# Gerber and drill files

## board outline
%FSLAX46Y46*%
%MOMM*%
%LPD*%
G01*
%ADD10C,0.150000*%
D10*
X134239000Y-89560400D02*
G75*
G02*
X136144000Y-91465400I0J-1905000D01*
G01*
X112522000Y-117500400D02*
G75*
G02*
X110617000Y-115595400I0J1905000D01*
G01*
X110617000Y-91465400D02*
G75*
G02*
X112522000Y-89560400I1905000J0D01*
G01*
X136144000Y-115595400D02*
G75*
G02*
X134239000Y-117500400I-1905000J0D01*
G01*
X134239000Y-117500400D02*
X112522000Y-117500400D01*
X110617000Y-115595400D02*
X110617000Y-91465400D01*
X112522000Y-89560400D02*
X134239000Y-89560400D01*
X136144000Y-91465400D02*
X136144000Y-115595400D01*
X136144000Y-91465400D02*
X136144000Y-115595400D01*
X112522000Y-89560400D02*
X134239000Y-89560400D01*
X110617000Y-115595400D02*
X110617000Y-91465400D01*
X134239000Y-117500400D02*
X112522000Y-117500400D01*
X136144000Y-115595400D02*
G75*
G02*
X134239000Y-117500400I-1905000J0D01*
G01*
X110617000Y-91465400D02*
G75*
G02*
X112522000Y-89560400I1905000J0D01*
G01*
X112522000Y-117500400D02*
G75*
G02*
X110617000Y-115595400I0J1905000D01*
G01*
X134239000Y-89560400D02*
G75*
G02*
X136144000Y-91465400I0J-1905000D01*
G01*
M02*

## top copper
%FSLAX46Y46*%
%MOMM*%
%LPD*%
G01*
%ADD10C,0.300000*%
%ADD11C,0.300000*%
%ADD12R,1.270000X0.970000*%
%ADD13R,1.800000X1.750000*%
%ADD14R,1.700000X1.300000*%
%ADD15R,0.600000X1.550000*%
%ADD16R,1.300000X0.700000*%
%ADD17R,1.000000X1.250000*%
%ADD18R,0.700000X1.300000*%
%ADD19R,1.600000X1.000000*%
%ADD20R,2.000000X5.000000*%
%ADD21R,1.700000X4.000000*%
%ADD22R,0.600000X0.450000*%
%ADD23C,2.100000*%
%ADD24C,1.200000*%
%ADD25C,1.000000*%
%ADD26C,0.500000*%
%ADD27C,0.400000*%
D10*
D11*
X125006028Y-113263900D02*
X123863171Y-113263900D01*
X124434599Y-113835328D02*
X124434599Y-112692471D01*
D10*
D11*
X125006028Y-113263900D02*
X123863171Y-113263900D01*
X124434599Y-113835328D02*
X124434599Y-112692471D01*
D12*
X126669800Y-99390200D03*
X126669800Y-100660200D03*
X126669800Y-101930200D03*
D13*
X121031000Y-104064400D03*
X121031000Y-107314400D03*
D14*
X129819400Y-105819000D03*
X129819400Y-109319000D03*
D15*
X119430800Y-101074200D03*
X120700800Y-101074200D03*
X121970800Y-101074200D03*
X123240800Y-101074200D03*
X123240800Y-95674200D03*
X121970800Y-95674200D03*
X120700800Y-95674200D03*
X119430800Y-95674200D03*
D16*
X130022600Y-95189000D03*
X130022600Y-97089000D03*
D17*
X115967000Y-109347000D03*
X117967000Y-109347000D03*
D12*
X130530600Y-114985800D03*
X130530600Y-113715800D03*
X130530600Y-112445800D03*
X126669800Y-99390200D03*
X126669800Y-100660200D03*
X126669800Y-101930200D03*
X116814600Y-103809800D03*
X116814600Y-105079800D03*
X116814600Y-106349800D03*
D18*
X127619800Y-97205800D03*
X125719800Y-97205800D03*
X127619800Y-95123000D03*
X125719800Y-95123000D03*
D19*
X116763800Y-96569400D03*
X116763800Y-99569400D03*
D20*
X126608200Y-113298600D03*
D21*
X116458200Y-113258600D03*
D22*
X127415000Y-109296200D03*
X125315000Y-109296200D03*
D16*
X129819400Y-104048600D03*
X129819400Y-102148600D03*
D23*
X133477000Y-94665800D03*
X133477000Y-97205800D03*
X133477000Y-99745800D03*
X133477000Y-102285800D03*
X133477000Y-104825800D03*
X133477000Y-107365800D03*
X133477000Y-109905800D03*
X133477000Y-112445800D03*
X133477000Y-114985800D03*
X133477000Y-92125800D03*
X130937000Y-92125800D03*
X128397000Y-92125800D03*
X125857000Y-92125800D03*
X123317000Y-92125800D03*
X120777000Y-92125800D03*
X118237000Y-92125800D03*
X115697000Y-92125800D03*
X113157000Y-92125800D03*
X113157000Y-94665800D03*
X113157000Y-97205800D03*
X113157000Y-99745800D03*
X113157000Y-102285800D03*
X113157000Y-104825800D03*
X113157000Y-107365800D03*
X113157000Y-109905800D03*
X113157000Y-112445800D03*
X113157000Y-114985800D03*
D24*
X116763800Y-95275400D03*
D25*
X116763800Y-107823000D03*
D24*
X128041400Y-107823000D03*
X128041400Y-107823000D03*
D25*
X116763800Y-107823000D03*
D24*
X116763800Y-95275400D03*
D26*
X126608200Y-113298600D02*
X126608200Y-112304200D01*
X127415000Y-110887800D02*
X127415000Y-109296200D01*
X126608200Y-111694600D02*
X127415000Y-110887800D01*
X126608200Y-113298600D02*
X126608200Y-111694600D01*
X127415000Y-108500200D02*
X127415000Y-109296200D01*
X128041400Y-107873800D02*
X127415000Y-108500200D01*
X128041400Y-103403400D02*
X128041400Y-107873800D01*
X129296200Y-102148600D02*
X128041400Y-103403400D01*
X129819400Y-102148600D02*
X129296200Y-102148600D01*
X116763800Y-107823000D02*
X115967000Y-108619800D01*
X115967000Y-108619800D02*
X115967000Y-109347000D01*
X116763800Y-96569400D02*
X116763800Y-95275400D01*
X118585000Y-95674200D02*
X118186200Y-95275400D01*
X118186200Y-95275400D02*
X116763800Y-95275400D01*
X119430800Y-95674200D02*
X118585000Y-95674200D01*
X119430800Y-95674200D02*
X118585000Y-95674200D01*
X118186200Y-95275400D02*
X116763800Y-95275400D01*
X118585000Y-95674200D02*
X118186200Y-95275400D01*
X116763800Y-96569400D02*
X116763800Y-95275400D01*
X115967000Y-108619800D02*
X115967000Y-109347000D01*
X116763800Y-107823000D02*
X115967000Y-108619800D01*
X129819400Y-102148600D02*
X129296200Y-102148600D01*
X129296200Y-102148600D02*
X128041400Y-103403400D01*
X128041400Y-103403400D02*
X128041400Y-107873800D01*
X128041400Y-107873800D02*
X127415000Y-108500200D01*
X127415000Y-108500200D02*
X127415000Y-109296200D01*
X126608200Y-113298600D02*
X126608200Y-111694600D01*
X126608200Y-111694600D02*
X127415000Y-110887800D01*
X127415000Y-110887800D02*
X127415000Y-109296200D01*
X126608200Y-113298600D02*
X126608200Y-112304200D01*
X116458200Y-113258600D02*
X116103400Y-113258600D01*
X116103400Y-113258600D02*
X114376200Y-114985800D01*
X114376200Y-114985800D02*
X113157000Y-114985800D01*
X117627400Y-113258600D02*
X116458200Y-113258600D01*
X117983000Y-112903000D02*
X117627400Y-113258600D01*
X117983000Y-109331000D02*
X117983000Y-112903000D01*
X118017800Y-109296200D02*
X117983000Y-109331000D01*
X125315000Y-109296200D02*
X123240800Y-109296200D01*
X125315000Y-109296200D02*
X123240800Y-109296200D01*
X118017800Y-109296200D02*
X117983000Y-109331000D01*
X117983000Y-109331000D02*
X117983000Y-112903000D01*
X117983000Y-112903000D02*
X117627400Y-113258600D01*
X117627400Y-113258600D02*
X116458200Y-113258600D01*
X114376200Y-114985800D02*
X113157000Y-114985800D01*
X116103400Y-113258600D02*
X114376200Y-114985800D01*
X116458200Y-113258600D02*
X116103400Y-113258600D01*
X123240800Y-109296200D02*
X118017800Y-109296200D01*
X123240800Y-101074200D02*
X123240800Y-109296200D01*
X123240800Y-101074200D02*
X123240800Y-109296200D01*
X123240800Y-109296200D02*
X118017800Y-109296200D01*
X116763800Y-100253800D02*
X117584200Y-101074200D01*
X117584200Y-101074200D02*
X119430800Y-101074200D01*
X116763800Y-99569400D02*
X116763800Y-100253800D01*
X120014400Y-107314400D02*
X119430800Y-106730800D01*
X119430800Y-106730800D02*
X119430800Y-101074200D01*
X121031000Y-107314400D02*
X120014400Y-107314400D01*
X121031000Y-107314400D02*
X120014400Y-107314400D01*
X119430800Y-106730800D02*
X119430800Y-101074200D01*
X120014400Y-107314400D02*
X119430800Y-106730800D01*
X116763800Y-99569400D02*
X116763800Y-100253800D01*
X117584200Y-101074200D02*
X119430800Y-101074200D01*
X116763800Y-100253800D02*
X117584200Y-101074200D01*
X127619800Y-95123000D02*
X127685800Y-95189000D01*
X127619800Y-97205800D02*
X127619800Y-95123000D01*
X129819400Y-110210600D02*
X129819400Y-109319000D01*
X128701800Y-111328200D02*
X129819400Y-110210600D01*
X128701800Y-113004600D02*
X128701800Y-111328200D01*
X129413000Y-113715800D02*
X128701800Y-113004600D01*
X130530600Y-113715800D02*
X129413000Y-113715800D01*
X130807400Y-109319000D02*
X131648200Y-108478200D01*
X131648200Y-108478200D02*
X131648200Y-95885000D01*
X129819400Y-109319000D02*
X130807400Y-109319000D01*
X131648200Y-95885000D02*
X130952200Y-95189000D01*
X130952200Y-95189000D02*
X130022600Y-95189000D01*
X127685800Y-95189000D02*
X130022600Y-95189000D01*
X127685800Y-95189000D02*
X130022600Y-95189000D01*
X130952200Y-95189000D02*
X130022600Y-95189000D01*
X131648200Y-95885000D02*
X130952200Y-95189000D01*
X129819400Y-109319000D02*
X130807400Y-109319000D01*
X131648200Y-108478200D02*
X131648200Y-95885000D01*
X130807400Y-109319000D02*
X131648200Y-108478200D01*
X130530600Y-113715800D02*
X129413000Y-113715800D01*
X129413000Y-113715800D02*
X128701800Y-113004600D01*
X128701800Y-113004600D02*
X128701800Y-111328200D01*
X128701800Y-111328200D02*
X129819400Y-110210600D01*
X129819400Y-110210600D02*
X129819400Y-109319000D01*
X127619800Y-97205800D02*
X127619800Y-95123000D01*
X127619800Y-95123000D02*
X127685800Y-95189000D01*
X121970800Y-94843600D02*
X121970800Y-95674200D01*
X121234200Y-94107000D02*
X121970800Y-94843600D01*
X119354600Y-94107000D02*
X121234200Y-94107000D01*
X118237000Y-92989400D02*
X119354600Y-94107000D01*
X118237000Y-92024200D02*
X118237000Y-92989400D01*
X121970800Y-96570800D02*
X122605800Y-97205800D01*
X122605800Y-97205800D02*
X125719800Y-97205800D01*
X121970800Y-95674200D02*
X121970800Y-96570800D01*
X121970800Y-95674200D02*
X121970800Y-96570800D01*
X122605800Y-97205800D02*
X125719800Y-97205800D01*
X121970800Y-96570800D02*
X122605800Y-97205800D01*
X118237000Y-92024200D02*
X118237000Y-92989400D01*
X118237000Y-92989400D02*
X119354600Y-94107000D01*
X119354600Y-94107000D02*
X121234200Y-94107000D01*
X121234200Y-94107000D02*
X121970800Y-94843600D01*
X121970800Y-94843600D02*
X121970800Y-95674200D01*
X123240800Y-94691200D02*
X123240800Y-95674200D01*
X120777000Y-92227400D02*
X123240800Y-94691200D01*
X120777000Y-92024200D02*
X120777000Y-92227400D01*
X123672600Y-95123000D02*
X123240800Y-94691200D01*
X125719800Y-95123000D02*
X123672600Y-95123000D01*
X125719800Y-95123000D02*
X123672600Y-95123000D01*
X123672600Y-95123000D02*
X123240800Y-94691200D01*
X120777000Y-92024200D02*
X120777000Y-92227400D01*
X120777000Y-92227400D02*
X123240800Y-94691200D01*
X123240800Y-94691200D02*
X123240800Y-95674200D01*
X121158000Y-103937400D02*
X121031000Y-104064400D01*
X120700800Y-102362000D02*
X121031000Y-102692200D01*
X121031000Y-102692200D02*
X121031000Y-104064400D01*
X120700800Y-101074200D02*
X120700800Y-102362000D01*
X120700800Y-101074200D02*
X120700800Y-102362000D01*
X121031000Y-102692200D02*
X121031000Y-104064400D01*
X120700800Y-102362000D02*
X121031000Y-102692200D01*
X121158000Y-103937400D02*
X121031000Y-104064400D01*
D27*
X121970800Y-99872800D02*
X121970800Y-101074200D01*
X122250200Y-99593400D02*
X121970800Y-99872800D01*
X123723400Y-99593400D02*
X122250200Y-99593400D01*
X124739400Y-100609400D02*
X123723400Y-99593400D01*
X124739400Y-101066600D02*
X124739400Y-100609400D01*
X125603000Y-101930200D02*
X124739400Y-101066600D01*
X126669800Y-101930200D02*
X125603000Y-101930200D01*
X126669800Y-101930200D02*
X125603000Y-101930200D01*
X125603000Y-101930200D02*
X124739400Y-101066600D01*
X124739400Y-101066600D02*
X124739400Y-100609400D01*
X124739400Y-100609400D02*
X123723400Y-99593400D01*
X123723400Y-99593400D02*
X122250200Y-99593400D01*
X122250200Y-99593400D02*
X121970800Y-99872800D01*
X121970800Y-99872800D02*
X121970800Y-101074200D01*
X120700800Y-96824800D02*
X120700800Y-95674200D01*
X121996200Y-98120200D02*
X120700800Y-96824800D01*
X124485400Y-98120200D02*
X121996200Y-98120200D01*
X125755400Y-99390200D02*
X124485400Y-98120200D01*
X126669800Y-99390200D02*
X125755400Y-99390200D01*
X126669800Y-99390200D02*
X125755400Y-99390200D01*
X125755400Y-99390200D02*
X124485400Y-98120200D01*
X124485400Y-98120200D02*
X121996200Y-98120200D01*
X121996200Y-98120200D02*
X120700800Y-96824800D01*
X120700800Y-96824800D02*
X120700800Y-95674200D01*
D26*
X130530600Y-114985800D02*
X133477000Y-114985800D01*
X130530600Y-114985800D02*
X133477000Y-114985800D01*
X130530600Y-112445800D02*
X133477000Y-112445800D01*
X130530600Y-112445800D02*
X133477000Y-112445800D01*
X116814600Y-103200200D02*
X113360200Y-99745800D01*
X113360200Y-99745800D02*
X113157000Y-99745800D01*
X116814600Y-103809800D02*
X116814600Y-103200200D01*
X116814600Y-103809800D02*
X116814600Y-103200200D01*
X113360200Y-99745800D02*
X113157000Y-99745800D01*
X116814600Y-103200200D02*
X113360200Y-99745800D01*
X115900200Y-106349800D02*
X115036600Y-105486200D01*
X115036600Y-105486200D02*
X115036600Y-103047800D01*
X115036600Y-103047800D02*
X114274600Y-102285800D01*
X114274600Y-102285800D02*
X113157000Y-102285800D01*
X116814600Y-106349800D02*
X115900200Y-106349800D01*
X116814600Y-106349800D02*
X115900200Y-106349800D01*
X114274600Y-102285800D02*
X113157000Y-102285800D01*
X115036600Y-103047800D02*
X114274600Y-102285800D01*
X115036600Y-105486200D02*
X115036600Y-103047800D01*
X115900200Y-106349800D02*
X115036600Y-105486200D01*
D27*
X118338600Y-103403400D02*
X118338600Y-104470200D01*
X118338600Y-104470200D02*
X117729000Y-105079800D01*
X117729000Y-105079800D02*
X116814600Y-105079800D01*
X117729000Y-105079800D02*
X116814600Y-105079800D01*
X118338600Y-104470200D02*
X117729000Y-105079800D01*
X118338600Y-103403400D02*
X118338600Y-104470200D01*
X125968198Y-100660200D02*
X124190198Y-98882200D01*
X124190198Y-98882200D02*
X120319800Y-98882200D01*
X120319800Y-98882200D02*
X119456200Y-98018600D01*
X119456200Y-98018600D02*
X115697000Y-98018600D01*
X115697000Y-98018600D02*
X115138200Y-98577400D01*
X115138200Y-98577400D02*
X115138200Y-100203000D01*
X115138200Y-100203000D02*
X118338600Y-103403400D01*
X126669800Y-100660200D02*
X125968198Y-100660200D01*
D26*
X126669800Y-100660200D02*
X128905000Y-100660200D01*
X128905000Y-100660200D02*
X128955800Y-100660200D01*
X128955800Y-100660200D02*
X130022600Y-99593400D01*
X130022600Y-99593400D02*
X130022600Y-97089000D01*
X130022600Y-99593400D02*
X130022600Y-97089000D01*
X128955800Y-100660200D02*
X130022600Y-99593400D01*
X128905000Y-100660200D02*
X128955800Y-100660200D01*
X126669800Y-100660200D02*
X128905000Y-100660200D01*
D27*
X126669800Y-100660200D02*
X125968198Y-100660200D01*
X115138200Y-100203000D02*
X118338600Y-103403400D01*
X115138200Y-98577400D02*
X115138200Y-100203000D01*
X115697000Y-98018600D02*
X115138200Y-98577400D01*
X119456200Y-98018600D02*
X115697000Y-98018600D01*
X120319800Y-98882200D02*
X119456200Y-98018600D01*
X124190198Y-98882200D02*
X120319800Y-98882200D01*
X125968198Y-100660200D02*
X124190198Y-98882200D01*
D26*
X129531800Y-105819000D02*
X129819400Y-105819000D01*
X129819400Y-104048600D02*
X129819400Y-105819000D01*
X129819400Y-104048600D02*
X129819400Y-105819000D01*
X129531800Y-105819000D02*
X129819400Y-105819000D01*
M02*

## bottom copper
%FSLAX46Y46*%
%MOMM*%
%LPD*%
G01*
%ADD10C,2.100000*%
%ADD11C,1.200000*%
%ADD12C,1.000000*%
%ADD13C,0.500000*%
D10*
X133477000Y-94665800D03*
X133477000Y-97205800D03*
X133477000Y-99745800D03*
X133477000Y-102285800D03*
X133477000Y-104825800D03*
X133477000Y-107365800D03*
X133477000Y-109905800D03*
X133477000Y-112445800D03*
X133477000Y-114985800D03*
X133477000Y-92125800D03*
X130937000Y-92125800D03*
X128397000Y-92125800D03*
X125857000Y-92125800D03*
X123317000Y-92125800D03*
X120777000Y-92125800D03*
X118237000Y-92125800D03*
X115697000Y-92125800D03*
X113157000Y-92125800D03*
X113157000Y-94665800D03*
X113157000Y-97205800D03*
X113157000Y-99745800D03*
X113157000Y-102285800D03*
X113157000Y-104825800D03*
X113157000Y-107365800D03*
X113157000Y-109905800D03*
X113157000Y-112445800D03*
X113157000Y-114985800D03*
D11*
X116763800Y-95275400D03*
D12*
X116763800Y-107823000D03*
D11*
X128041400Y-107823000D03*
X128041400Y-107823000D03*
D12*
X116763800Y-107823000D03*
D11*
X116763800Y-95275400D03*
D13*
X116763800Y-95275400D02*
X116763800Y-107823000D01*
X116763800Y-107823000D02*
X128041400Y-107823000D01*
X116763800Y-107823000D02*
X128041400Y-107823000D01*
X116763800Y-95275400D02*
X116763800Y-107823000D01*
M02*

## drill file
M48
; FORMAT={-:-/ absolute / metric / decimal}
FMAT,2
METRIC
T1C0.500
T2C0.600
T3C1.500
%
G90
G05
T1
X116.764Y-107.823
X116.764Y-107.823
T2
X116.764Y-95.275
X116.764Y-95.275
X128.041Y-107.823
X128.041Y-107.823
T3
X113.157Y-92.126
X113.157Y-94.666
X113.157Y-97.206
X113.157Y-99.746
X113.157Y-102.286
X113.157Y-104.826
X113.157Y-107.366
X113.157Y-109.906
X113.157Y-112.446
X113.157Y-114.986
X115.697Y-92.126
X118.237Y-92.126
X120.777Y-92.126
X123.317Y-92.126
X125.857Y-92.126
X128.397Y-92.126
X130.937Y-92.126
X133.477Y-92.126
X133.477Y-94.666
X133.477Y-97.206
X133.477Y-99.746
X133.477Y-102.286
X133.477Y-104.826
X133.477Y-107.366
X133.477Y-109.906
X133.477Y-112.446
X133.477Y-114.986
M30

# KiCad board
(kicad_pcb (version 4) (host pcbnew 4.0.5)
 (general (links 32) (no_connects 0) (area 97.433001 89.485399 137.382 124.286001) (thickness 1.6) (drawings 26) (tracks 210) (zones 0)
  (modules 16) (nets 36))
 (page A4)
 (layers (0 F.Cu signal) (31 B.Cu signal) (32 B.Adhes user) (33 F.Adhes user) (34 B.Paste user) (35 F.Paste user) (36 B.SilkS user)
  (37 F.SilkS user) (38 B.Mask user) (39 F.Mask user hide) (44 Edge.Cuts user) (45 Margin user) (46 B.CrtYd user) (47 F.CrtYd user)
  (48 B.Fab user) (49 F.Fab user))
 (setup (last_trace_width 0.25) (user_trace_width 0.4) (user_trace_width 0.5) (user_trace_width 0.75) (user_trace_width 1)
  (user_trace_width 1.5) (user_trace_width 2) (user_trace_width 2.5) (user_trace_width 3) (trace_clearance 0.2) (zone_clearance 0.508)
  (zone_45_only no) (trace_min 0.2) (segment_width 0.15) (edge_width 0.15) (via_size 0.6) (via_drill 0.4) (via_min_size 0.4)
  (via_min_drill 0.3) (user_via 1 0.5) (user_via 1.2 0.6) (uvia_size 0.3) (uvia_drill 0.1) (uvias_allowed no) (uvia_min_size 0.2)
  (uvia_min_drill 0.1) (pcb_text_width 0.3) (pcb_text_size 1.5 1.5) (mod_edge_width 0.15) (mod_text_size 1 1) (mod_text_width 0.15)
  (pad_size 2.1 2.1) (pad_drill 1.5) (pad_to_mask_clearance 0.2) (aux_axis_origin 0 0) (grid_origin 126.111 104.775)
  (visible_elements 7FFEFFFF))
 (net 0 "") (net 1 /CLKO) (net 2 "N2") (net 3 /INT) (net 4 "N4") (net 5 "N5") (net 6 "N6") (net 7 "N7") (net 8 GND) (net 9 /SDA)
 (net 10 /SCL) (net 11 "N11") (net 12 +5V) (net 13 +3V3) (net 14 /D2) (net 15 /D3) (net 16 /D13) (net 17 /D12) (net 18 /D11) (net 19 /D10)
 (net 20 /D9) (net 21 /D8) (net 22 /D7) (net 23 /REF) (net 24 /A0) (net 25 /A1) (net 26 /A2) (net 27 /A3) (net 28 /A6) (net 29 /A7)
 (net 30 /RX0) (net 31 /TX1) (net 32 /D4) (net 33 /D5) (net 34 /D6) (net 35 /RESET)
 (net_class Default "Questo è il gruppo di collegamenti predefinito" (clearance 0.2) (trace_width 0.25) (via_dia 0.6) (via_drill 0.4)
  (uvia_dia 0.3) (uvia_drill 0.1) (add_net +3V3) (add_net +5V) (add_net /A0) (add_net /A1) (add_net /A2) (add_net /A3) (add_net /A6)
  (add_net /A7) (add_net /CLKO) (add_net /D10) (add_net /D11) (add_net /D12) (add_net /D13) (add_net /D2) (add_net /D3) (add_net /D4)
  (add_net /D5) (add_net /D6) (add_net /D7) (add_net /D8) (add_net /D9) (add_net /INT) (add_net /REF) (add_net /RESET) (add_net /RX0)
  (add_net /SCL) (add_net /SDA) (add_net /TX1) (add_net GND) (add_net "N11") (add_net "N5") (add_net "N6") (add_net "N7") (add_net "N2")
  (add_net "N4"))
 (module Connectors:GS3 (layer F.Cu) (at 126.6698 100.6602)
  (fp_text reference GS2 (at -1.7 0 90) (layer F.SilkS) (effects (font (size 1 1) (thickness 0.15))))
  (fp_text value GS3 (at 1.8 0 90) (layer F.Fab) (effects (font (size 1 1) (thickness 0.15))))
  (pad 1 smd rect (at 0 -1.27) (size 1.27 0.97) (layers F.Cu F.Paste F.Mask) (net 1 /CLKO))
  (pad 2 smd rect (at 0 0) (size 1.27 0.97) (layers F.Cu F.Paste F.Mask) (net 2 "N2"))
  (pad 3 smd rect (at 0 1.27) (size 1.27 0.97) (layers F.Cu F.Paste F.Mask) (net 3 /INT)))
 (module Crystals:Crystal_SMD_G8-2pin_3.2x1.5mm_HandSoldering (layer F.Cu) (at 121.031 105.6894 270)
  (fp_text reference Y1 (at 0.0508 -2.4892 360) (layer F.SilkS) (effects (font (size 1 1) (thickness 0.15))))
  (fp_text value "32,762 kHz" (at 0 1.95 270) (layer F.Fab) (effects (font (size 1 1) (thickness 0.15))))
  (pad 1 smd rect (at -1.625 0 270) (size 1.75 1.8) (layers F.Cu F.Paste F.Mask) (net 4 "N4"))
  (pad 2 smd rect (at 1.625 0 270) (size 1.75 1.8) (layers F.Cu F.Paste F.Mask) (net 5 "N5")))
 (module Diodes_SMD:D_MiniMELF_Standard (layer F.Cu) (at 129.8194 107.569 270)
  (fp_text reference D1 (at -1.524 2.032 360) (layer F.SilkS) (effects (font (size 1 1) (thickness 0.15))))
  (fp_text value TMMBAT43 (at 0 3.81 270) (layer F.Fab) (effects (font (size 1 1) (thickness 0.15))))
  (pad 1 smd rect (at -1.75 0 270) (size 1.3 1.7) (layers F.Cu F.Paste F.Mask) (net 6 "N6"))
  (pad 2 smd rect (at 1.75 0 270) (size 1.3 1.7) (layers F.Cu F.Paste F.Mask) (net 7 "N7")))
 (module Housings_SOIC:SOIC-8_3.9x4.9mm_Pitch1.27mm (layer F.Cu) (at 121.3358 98.3742 90)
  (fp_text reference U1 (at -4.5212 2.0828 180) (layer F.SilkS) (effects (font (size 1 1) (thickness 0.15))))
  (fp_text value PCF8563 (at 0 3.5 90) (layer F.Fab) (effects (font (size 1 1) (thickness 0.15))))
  (pad 1 smd rect (at -2.7 -1.905 90) (size 1.55 0.6) (layers F.Cu F.Paste F.Mask) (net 5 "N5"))
  (pad 2 smd rect (at -2.7 -0.635 90) (size 1.55 0.6) (layers F.Cu F.Paste F.Mask) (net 4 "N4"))
  (pad 3 smd rect (at -2.7 0.635 90) (size 1.55 0.6) (layers F.Cu F.Paste F.Mask) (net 3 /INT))
  (pad 4 smd rect (at -2.7 1.905 90) (size 1.55 0.6) (layers F.Cu F.Paste F.Mask) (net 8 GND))
  (pad 5 smd rect (at 2.7 1.905 90) (size 1.55 0.6) (layers F.Cu F.Paste F.Mask) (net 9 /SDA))
  (pad 6 smd rect (at 2.7 0.635 90) (size 1.55 0.6) (layers F.Cu F.Paste F.Mask) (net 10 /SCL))
  (pad 7 smd rect (at 2.7 -0.635 90) (size 1.55 0.6) (layers F.Cu F.Paste F.Mask) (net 1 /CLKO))
  (pad 8 smd rect (at 2.7 -1.905 90) (size 1.55 0.6) (layers F.Cu F.Paste F.Mask) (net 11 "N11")))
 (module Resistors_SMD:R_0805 (layer F.Cu) (at 130.0226 96.139 270)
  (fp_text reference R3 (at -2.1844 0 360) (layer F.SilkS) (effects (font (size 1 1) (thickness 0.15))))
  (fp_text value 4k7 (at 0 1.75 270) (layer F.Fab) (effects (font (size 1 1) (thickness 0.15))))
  (pad 1 smd rect (at -0.95 0 270) (size 0.7 1.3) (layers F.Cu F.Paste F.Mask) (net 7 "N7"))
  (pad 2 smd rect (at 0.95 0 270) (size 0.7 1.3) (layers F.Cu F.Paste F.Mask) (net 2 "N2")))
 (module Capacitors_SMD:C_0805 (layer F.Cu) (at 116.967 109.347)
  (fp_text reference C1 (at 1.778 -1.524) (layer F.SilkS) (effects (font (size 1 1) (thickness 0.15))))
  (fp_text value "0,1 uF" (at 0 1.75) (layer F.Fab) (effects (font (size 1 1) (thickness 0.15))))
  (pad 1 smd rect (at -1 0) (size 1 1.25) (layers F.Cu F.Paste F.Mask) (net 11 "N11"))
  (pad 2 smd rect (at 1 0) (size 1 1.25) (layers F.Cu F.Paste F.Mask) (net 8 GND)))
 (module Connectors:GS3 (layer F.Cu) (at 130.5306 113.7158 180)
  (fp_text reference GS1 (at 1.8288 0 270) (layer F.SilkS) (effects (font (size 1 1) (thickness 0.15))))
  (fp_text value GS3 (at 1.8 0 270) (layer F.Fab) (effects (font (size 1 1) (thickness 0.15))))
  (pad 1 smd rect (at 0 -1.27 180) (size 1.27 0.97) (layers F.Cu F.Paste F.Mask) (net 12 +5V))
  (pad 2 smd rect (at 0 0 180) (size 1.27 0.97) (layers F.Cu F.Paste F.Mask) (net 7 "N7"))
  (pad 3 smd rect (at 0 1.27 180) (size 1.27 0.97) (layers F.Cu F.Paste F.Mask) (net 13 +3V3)))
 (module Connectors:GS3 (layer F.Cu) (at 126.6698 100.6602)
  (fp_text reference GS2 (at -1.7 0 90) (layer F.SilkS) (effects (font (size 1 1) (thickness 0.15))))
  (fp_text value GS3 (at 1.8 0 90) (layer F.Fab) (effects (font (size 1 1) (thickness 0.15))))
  (pad 1 smd rect (at 0 -1.27) (size 1.27 0.97) (layers F.Cu F.Paste F.Mask) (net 1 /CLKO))
  (pad 2 smd rect (at 0 0) (size 1.27 0.97) (layers F.Cu F.Paste F.Mask) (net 2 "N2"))
  (pad 3 smd rect (at 0 1.27) (size 1.27 0.97) (layers F.Cu F.Paste F.Mask) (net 3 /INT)))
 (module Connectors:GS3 (layer F.Cu) (at 116.8146 105.0798)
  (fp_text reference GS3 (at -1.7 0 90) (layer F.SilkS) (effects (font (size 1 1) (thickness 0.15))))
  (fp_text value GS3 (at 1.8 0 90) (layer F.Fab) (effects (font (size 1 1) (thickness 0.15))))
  (pad 1 smd rect (at 0 -1.27) (size 1.27 0.97) (layers F.Cu F.Paste F.Mask) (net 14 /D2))
  (pad 2 smd rect (at 0 0) (size 1.27 0.97) (layers F.Cu F.Paste F.Mask) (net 2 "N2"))
  (pad 3 smd rect (at 0 1.27) (size 1.27 0.97) (layers F.Cu F.Paste F.Mask) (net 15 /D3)))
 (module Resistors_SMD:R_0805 (layer F.Cu) (at 126.6698 97.2058 180)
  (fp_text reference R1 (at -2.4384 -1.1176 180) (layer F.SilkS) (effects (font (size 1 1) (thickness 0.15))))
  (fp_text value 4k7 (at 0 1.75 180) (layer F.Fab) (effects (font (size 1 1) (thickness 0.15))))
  (pad 1 smd rect (at -0.95 0 180) (size 0.7 1.3) (layers F.Cu F.Paste F.Mask) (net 7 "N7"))
  (pad 2 smd rect (at 0.95 0 180) (size 0.7 1.3) (layers F.Cu F.Paste F.Mask) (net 10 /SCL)))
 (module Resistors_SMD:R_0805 (layer F.Cu) (at 126.6698 95.123 180)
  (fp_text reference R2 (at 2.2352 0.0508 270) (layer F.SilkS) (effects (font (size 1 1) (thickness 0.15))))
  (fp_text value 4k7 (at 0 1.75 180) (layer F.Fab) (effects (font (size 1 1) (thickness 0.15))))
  (pad 1 smd rect (at -0.95 0 180) (size 0.7 1.3) (layers F.Cu F.Paste F.Mask) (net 7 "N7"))
  (pad 2 smd rect (at 0.95 0 180) (size 0.7 1.3) (layers F.Cu F.Paste F.Mask) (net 9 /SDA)))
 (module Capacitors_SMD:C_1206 (layer F.Cu) (at 116.7638 98.0694 270)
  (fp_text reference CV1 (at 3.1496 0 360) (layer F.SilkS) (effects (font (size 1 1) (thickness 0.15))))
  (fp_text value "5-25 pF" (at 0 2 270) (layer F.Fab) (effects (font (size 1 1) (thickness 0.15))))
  (pad 1 smd rect (at -1.5 0 270) (size 1 1.6) (layers F.Cu F.Paste F.Mask) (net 11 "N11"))
  (pad 2 smd rect (at 1.5 0 270) (size 1 1.6) (layers F.Cu F.Paste F.Mask) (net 5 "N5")))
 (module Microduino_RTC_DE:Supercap (layer F.Cu) (at 121.4882 113.2586 180)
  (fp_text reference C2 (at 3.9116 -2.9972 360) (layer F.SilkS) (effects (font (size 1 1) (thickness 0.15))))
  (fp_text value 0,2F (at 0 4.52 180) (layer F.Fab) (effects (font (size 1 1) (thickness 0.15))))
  (pad 1 smd rect (at -5.12 -0.04 180) (size 2 5) (layers F.Cu F.Paste F.Mask) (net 11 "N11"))
  (pad 2 smd rect (at 5.03 0 180) (size 1.7 4) (layers F.Cu F.Mask) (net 8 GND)))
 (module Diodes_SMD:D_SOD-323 (layer F.Cu) (at 126.365 109.2962 180)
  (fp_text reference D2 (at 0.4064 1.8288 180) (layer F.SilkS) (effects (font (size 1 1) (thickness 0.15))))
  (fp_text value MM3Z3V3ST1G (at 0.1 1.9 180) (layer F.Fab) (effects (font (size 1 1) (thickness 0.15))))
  (pad 1 smd rect (at -1.05 0 180) (size 0.6 0.45) (layers F.Cu F.Paste F.Mask) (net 11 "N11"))
  (pad 2 smd rect (at 1.05 0 180) (size 0.6 0.45) (layers F.Cu F.Paste F.Mask) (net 8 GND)))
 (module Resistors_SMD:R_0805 (layer F.Cu) (at 129.8194 103.0986 90)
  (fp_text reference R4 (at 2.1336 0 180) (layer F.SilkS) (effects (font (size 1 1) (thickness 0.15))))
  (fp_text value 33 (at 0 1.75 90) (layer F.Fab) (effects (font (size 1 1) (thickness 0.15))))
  (pad 1 smd rect (at -0.95 0 90) (size 0.7 1.3) (layers F.Cu F.Paste F.Mask) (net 6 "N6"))
  (pad 2 smd rect (at 0.95 0 90) (size 0.7 1.3) (layers F.Cu F.Paste F.Mask) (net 11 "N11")))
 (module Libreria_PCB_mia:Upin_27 (layer B.Cu) (at 133.477 114.9858 180)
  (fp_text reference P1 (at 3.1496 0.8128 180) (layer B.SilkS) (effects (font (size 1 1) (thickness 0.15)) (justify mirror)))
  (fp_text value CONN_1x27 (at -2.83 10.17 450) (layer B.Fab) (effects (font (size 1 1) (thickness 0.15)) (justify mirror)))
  (pad 9 thru_hole circle (at 0 20.32 180) (size 2.1 2.1) (drill 1.5) (layers *.Cu *.Mask) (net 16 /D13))
  (pad 8 thru_hole circle (at 0 17.78 180) (size 2.1 2.1) (drill 1.5) (layers *.Cu *.Mask) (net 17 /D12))
  (pad 7 thru_hole circle (at 0 15.24 180) (size 2.1 2.1) (drill 1.5) (layers *.Cu *.Mask) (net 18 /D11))
  (pad 6 thru_hole circle (at 0 12.7 180) (size 2.1 2.1) (drill 1.5) (layers *.Cu *.Mask) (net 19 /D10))
  (pad 5 thru_hole circle (at 0 10.16 180) (size 2.1 2.1) (drill 1.5) (layers *.Cu *.Mask) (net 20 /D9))
  (pad 4 thru_hole circle (at 0 7.62 180) (size 2.1 2.1) (drill 1.5) (layers *.Cu *.Mask) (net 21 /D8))
  (pad 3 thru_hole circle (at 0 5.08 180) (size 2.1 2.1) (drill 1.5) (layers *.Cu *.Mask) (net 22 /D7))
  (pad 2 thru_hole circle (at 0 2.54 180) (size 2.1 2.1) (drill 1.5) (layers *.Cu *.Mask) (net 13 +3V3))
  (pad 1 thru_hole circle (at 0 0 180) (size 2.1 2.1) (drill 1.5) (layers *.Cu *.Mask) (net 12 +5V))
  (pad 10 thru_hole circle (at 0 22.86 180) (size 2.1 2.1) (drill 1.5) (layers *.Cu *.Mask) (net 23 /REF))
  (pad 11 thru_hole circle (at 2.54 22.86 180) (size 2.1 2.1) (drill 1.5) (layers *.Cu *.Mask) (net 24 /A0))
  (pad 12 thru_hole circle (at 5.08 22.86 180) (size 2.1 2.1) (drill 1.5) (layers *.Cu *.Mask) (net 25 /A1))
  (pad 13 thru_hole circle (at 7.62 22.86 180) (size 2.1 2.1) (drill 1.5) (layers *.Cu *.Mask) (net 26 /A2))
  (pad 14 thru_hole circle (at 10.16 22.86 180) (size 2.1 2.1) (drill 1.5) (layers *.Cu *.Mask) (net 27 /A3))
  (pad 15 thru_hole circle (at 12.7 22.86 180) (size 2.1 2.1) (drill 1.5) (layers *.Cu *.Mask) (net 9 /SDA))
  (pad 16 thru_hole circle (at 15.24 22.86 180) (size 2.1 2.1) (drill 1.5) (layers *.Cu *.Mask) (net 10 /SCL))
  (pad 17 thru_hole circle (at 17.78 22.86 180) (size 2.1 2.1) (drill 1.5) (layers *.Cu *.Mask) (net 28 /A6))
  (pad 18 thru_hole circle (at 20.32 22.86 180) (size 2.1 2.1) (drill 1.5) (layers *.Cu *.Mask) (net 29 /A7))
  (pad 19 thru_hole circle (at 20.32 20.32 180) (size 2.1 2.1) (drill 1.5) (layers *.Cu *.Mask) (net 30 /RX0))
  (pad 20 thru_hole circle (at 20.32 17.78 180) (size 2.1 2.1) (drill 1.5) (layers *.Cu *.Mask) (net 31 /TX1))
  (pad 21 thru_hole circle (at 20.32 15.24 180) (size 2.1 2.1) (drill 1.5) (layers *.Cu *.Mask) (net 14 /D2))
  (pad 22 thru_hole circle (at 20.32 12.7 180) (size 2.1 2.1) (drill 1.5) (layers *.Cu *.Mask) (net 15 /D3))
  (pad 23 thru_hole circle (at 20.32 10.16 180) (size 2.1 2.1) (drill 1.5) (layers *.Cu *.Mask) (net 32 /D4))
  (pad 24 thru_hole circle (at 20.32 7.62 180) (size 2.1 2.1) (drill 1.5) (layers *.Cu *.Mask) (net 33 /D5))
  (pad 25 thru_hole circle (at 20.32 5.08 180) (size 2.1 2.1) (drill 1.5) (layers *.Cu *.Mask) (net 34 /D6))
  (pad 26 thru_hole circle (at 20.32 2.54 180) (size 2.1 2.1) (drill 1.5) (layers *.Cu *.Mask) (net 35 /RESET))
  (pad 27 thru_hole circle (at 20.32 0 180) (size 2.1 2.1) (drill 1.5) (layers *.Cu *.Mask) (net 8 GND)))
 (gr_arc (start 134.239 91.4654) (end 134.239 89.5604) (angle 90) (layer Edge.Cuts) (width 0.15))
 (gr_arc (start 112.522 115.5954) (end 112.522 117.5004) (angle 90) (layer Edge.Cuts) (width 0.15))
 (gr_arc (start 112.522 91.4654) (end 110.617 91.4654) (angle 90) (layer Edge.Cuts) (width 0.15))
 (gr_arc (start 134.239 115.5954) (end 136.144 115.5954) (angle 90) (layer Edge.Cuts) (width 0.15))
 (gr_line (start 134.239 117.5004) (end 112.522 117.5004) (angle 90) (layer Edge.Cuts) (width 0.15))
 (gr_line (start 110.617 115.5954) (end 110.617 91.4654) (angle 90) (layer Edge.Cuts) (width 0.15))
 (gr_line (start 112.522 89.5604) (end 134.239 89.5604) (angle 90) (layer Edge.Cuts) (width 0.15))
 (gr_line (start 136.144 91.4654) (end 136.144 115.5954) (angle 90) (layer Edge.Cuts) (width 0.15))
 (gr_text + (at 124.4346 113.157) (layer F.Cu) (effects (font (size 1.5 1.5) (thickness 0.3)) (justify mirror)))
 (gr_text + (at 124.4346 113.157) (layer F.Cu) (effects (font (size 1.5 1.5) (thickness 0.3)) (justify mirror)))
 (gr_line (start 136.144 91.4654) (end 136.144 115.5954) (angle 90) (layer Edge.Cuts) (width 0.15))
 (gr_line (start 112.522 89.5604) (end 134.239 89.5604) (angle 90) (layer Edge.Cuts) (width 0.15))
 (gr_line (start 110.617 115.5954) (end 110.617 91.4654) (angle 90) (layer Edge.Cuts) (width 0.15))
 (gr_line (start 134.239 117.5004) (end 112.522 117.5004) (angle 90) (layer Edge.Cuts) (width 0.15))
 (gr_arc (start 134.239 115.5954) (end 136.144 115.5954) (angle 90) (layer Edge.Cuts) (width 0.15))
 (gr_arc (start 112.522 91.4654) (end 110.617 91.4654) (angle 90) (layer Edge.Cuts) (width 0.15))
 (gr_arc (start 112.522 115.5954) (end 112.522 117.5004) (angle 90) (layer Edge.Cuts) (width 0.15))
 (gr_arc (start 134.239 91.4654) (end 134.239 89.5604) (angle 90) (layer Edge.Cuts) (width 0.15))
 (segment (start 126.6082 113.2986) (end 126.6082 112.3042) (width 0.5) (layer F.Cu) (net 11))
 (segment (start 127.415 110.8878) (end 127.415 109.2962) (width 0.5) (layer F.Cu) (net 11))
 (segment (start 126.6082 111.6946) (end 127.415 110.8878) (width 0.5) (layer F.Cu) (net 11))
 (segment (start 126.6082 113.2986) (end 126.6082 111.6946) (width 0.5) (layer F.Cu) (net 11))
 (segment (start 127.415 108.5002) (end 127.415 109.2962) (width 0.5) (layer F.Cu) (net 11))
 (segment (start 128.0414 107.8738) (end 127.415 108.5002) (width 0.5) (layer F.Cu) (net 11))
 (segment (start 128.0414 103.4034) (end 128.0414 107.8738) (width 0.5) (layer F.Cu) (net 11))
 (segment (start 129.2962 102.1486) (end 128.0414 103.4034) (width 0.5) (layer F.Cu) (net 11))
 (segment (start 129.8194 102.1486) (end 129.2962 102.1486) (width 0.5) (layer F.Cu) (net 11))
 (via (at 116.7638 95.2754) (size 1.2) (drill 0.6) (layers F.Cu B.Cu) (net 11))
 (segment (start 116.7638 95.2754) (end 116.7638 107.823) (width 0.5) (layer B.Cu) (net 11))
 (via (at 116.7638 107.823) (size 1) (drill 0.5) (layers F.Cu B.Cu) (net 11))
 (segment (start 116.7638 107.823) (end 115.967 108.6198) (width 0.5) (layer F.Cu) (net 11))
 (segment (start 115.967 108.6198) (end 115.967 109.347) (width 0.5) (layer F.Cu) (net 11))
 (segment (start 116.7638 96.5694) (end 116.7638 95.2754) (width 0.5) (layer F.Cu) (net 11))
 (segment (start 118.585 95.6742) (end 118.1862 95.2754) (width 0.5) (layer F.Cu) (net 11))
 (segment (start 118.1862 95.2754) (end 116.7638 95.2754) (width 0.5) (layer F.Cu) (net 11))
 (segment (start 119.4308 95.6742) (end 118.585 95.6742) (width 0.5) (layer F.Cu) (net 11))
 (via (at 128.0414 107.823) (size 1.2) (drill 0.6) (layers F.Cu B.Cu) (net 11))
 (segment (start 116.7638 107.823) (end 128.0414 107.823) (width 0.5) (layer B.Cu) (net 11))
 (segment (start 116.7638 107.823) (end 128.0414 107.823) (width 0.5) (layer B.Cu) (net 11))
 (via (at 128.0414 107.823) (size 1.2) (drill 0.6) (layers F.Cu B.Cu) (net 11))
 (segment (start 119.4308 95.6742) (end 118.585 95.6742) (width 0.5) (layer F.Cu) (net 11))
 (segment (start 118.1862 95.2754) (end 116.7638 95.2754) (width 0.5) (layer F.Cu) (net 11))
 (segment (start 118.585 95.6742) (end 118.1862 95.2754) (width 0.5) (layer F.Cu) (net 11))
 (segment (start 116.7638 96.5694) (end 116.7638 95.2754) (width 0.5) (layer F.Cu) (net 11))
 (segment (start 115.967 108.6198) (end 115.967 109.347) (width 0.5) (layer F.Cu) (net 11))
 (segment (start 116.7638 107.823) (end 115.967 108.6198) (width 0.5) (layer F.Cu) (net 11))
 (via (at 116.7638 107.823) (size 1) (drill 0.5) (layers F.Cu B.Cu) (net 11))
 (segment (start 116.7638 95.2754) (end 116.7638 107.823) (width 0.5) (layer B.Cu) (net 11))
 (via (at 116.7638 95.2754) (size 1.2) (drill 0.6) (layers F.Cu B.Cu) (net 11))
 (segment (start 129.8194 102.1486) (end 129.2962 102.1486) (width 0.5) (layer F.Cu) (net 11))
 (segment (start 129.2962 102.1486) (end 128.0414 103.4034) (width 0.5) (layer F.Cu) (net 11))
 (segment (start 128.0414 103.4034) (end 128.0414 107.8738) (width 0.5) (layer F.Cu) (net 11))
 (segment (start 128.0414 107.8738) (end 127.415 108.5002) (width 0.5) (layer F.Cu) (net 11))
 (segment (start 127.415 108.5002) (end 127.415 109.2962) (width 0.5) (layer F.Cu) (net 11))
 (segment (start 126.6082 113.2986) (end 126.6082 111.6946) (width 0.5) (layer F.Cu) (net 11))
 (segment (start 126.6082 111.6946) (end 127.415 110.8878) (width 0.5) (layer F.Cu) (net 11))
 (segment (start 127.415 110.8878) (end 127.415 109.2962) (width 0.5) (layer F.Cu) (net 11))
 (segment (start 126.6082 113.2986) (end 126.6082 112.3042) (width 0.5) (layer F.Cu) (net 11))
 (segment (start 116.4582 113.2586) (end 116.1034 113.2586) (width 0.5) (layer F.Cu) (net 8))
 (segment (start 116.1034 113.2586) (end 114.3762 114.9858) (width 0.5) (layer F.Cu) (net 8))
 (segment (start 114.3762 114.9858) (end 113.157 114.9858) (width 0.5) (layer F.Cu) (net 8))
 (segment (start 117.6274 113.2586) (end 116.4582 113.2586) (width 0.5) (layer F.Cu) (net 8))
 (segment (start 117.983 112.903) (end 117.6274 113.2586) (width 0.5) (layer F.Cu) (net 8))
 (segment (start 117.983 109.331) (end 117.983 112.903) (width 0.5) (layer F.Cu) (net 8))
 (segment (start 118.0178 109.2962) (end 117.983 109.331) (width 0.5) (layer F.Cu) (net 8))
 (segment (start 125.315 109.2962) (end 123.2408 109.2962) (width 0.5) (layer F.Cu) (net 8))
 (segment (start 125.315 109.2962) (end 123.2408 109.2962) (width 0.5) (layer F.Cu) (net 8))
 (segment (start 118.0178 109.2962) (end 117.983 109.331) (width 0.5) (layer F.Cu) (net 8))
 (segment (start 117.983 109.331) (end 117.983 112.903) (width 0.5) (layer F.Cu) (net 8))
 (segment (start 117.983 112.903) (end 117.6274 113.2586) (width 0.5) (layer F.Cu) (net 8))
 (segment (start 117.6274 113.2586) (end 116.4582 113.2586) (width 0.5) (layer F.Cu) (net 8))
 (segment (start 114.3762 114.9858) (end 113.157 114.9858) (width 0.5) (layer F.Cu) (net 8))
 (segment (start 116.1034 113.2586) (end 114.3762 114.9858) (width 0.5) (layer F.Cu) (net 8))
 (segment (start 116.4582 113.2586) (end 116.1034 113.2586) (width 0.5) (layer F.Cu) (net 8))
 (segment (start 123.2408 109.2962) (end 118.0178 109.2962) (width 0.5) (layer F.Cu) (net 8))
 (segment (start 123.2408 101.0742) (end 123.2408 109.2962) (width 0.5) (layer F.Cu) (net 8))
 (segment (start 123.2408 101.0742) (end 123.2408 109.2962) (width 0.5) (layer F.Cu) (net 8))
 (segment (start 123.2408 109.2962) (end 118.0178 109.2962) (width 0.5) (layer F.Cu) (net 8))
 (segment (start 116.7638 100.2538) (end 117.5842 101.0742) (width 0.5) (layer F.Cu) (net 5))
 (segment (start 117.5842 101.0742) (end 119.4308 101.0742) (width 0.5) (layer F.Cu) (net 5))
 (segment (start 116.7638 99.5694) (end 116.7638 100.2538) (width 0.5) (layer F.Cu) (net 5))
 (segment (start 120.0144 107.3144) (end 119.4308 106.7308) (width 0.5) (layer F.Cu) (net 5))
 (segment (start 119.4308 106.7308) (end 119.4308 101.0742) (width 0.5) (layer F.Cu) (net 5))
 (segment (start 121.031 107.3144) (end 120.0144 107.3144) (width 0.5) (layer F.Cu) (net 5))
 (segment (start 121.031 107.3144) (end 120.0144 107.3144) (width 0.5) (layer F.Cu) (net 5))
 (segment (start 119.4308 106.7308) (end 119.4308 101.0742) (width 0.5) (layer F.Cu) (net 5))
 (segment (start 120.0144 107.3144) (end 119.4308 106.7308) (width 0.5) (layer F.Cu) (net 5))
 (segment (start 116.7638 99.5694) (end 116.7638 100.2538) (width 0.5) (layer F.Cu) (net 5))
 (segment (start 117.5842 101.0742) (end 119.4308 101.0742) (width 0.5) (layer F.Cu) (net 5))
 (segment (start 116.7638 100.2538) (end 117.5842 101.0742) (width 0.5) (layer F.Cu) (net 5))
 (segment (start 127.6198 95.123) (end 127.6858 95.189) (width 0.5) (layer F.Cu) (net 7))
 (segment (start 127.6198 97.2058) (end 127.6198 95.123) (width 0.5) (layer F.Cu) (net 7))
 (segment (start 129.8194 110.2106) (end 129.8194 109.319) (width 0.5) (layer F.Cu) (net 7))
 (segment (start 128.7018 111.3282) (end 129.8194 110.2106) (width 0.5) (layer F.Cu) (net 7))
 (segment (start 128.7018 113.0046) (end 128.7018 111.3282) (width 0.5) (layer F.Cu) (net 7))
 (segment (start 129.413 113.7158) (end 128.7018 113.0046) (width 0.5) (layer F.Cu) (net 7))
 (segment (start 130.5306 113.7158) (end 129.413 113.7158) (width 0.5) (layer F.Cu) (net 7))
 (segment (start 130.8074 109.319) (end 131.6482 108.4782) (width 0.5) (layer F.Cu) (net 7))
 (segment (start 131.6482 108.4782) (end 131.6482 95.885) (width 0.5) (layer F.Cu) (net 7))
 (segment (start 129.8194 109.319) (end 130.8074 109.319) (width 0.5) (layer F.Cu) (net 7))
 (segment (start 131.6482 95.885) (end 130.9522 95.189) (width 0.5) (layer F.Cu) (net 7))
 (segment (start 130.9522 95.189) (end 130.0226 95.189) (width 0.5) (layer F.Cu) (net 7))
 (segment (start 127.6858 95.189) (end 130.0226 95.189) (width 0.5) (layer F.Cu) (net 7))
 (segment (start 127.6858 95.189) (end 130.0226 95.189) (width 0.5) (layer F.Cu) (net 7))
 (segment (start 130.9522 95.189) (end 130.0226 95.189) (width 0.5) (layer F.Cu) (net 7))
 (segment (start 131.6482 95.885) (end 130.9522 95.189) (width 0.5) (layer F.Cu) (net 7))
 (segment (start 129.8194 109.319) (end 130.8074 109.319) (width 0.5) (layer F.Cu) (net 7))
 (segment (start 131.6482 108.4782) (end 131.6482 95.885) (width 0.5) (layer F.Cu) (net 7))
 (segment (start 130.8074 109.319) (end 131.6482 108.4782) (width 0.5) (layer F.Cu) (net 7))
 (segment (start 130.5306 113.7158) (end 129.413 113.7158) (width 0.5) (layer F.Cu) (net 7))
 (segment (start 129.413 113.7158) (end 128.7018 113.0046) (width 0.5) (layer F.Cu) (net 7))
 (segment (start 128.7018 113.0046) (end 128.7018 111.3282) (width 0.5) (layer F.Cu) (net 7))
 (segment (start 128.7018 111.3282) (end 129.8194 110.2106) (width 0.5) (layer F.Cu) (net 7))
 (segment (start 129.8194 110.2106) (end 129.8194 109.319) (width 0.5) (layer F.Cu) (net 7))
 (segment (start 127.6198 97.2058) (end 127.6198 95.123) (width 0.5) (layer F.Cu) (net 7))
 (segment (start 127.6198 95.123) (end 127.6858 95.189) (width 0.5) (layer F.Cu) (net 7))
 (segment (start 121.9708 94.8436) (end 121.9708 95.6742) (width 0.5) (layer F.Cu) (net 10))
 (segment (start 121.2342 94.107) (end 121.9708 94.8436) (width 0.5) (layer F.Cu) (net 10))
 (segment (start 119.3546 94.107) (end 121.2342 94.107) (width 0.5) (layer F.Cu) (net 10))
 (segment (start 118.237 92.9894) (end 119.3546 94.107) (width 0.5) (layer F.Cu) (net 10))
 (segment (start 118.237 92.0242) (end 118.237 92.9894) (width 0.5) (layer F.Cu) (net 10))
 (segment (start 121.9708 96.5708) (end 122.6058 97.2058) (width 0.5) (layer F.Cu) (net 10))
 (segment (start 122.6058 97.2058) (end 125.7198 97.2058) (width 0.5) (layer F.Cu) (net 10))
 (segment (start 121.9708 95.6742) (end 121.9708 96.5708) (width 0.5) (layer F.Cu) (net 10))
 (segment (start 121.9708 95.6742) (end 121.9708 96.5708) (width 0.5) (layer F.Cu) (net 10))
 (segment (start 122.6058 97.2058) (end 125.7198 97.2058) (width 0.5) (layer F.Cu) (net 10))
 (segment (start 121.9708 96.5708) (end 122.6058 97.2058) (width 0.5) (layer F.Cu) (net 10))
 (segment (start 118.237 92.0242) (end 118.237 92.9894) (width 0.5) (layer F.Cu) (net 10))
 (segment (start 118.237 92.9894) (end 119.3546 94.107) (width 0.5) (layer F.Cu) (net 10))
 (segment (start 119.3546 94.107) (end 121.2342 94.107) (width 0.5) (layer F.Cu) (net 10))
 (segment (start 121.2342 94.107) (end 121.9708 94.8436) (width 0.5) (layer F.Cu) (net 10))
 (segment (start 121.9708 94.8436) (end 121.9708 95.6742) (width 0.5) (layer F.Cu) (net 10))
 (segment (start 123.2408 94.6912) (end 123.2408 95.6742) (width 0.5) (layer F.Cu) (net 9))
 (segment (start 120.777 92.2274) (end 123.2408 94.6912) (width 0.5) (layer F.Cu) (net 9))
 (segment (start 120.777 92.0242) (end 120.777 92.2274) (width 0.5) (layer F.Cu) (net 9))
 (segment (start 123.6726 95.123) (end 123.2408 94.6912) (width 0.5) (layer F.Cu) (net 9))
 (segment (start 125.7198 95.123) (end 123.6726 95.123) (width 0.5) (layer F.Cu) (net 9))
 (segment (start 125.7198 95.123) (end 123.6726 95.123) (width 0.5) (layer F.Cu) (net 9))
 (segment (start 123.6726 95.123) (end 123.2408 94.6912) (width 0.5) (layer F.Cu) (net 9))
 (segment (start 120.777 92.0242) (end 120.777 92.2274) (width 0.5) (layer F.Cu) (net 9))
 (segment (start 120.777 92.2274) (end 123.2408 94.6912) (width 0.5) (layer F.Cu) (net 9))
 (segment (start 123.2408 94.6912) (end 123.2408 95.6742) (width 0.5) (layer F.Cu) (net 9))
 (segment (start 121.158 103.9374) (end 121.031 104.0644) (width 0.5) (layer F.Cu) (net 4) (status 30))
 (segment (start 120.7008 102.362) (end 121.031 102.6922) (width 0.5) (layer F.Cu) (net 4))
 (segment (start 121.031 102.6922) (end 121.031 104.0644) (width 0.5) (layer F.Cu) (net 4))
 (segment (start 120.7008 101.0742) (end 120.7008 102.362) (width 0.5) (layer F.Cu) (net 4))
 (segment (start 120.7008 101.0742) (end 120.7008 102.362) (width 0.5) (layer F.Cu) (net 4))
 (segment (start 121.031 102.6922) (end 121.031 104.0644) (width 0.5) (layer F.Cu) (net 4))
 (segment (start 120.7008 102.362) (end 121.031 102.6922) (width 0.5) (layer F.Cu) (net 4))
 (segment (start 121.158 103.9374) (end 121.031 104.0644) (width 0.5) (layer F.Cu) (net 4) (status 30))
 (segment (start 121.9708 99.8728) (end 121.9708 101.0742) (width 0.4) (layer F.Cu) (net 3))
 (segment (start 122.2502 99.5934) (end 121.9708 99.8728) (width 0.4) (layer F.Cu) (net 3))
 (segment (start 123.7234 99.5934) (end 122.2502 99.5934) (width 0.4) (layer F.Cu) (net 3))
 (segment (start 124.7394 100.6094) (end 123.7234 99.5934) (width 0.4) (layer F.Cu) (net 3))
 (segment (start 124.7394 101.0666) (end 124.7394 100.6094) (width 0.4) (layer F.Cu) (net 3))
 (segment (start 125.603 101.9302) (end 124.7394 101.0666) (width 0.4) (layer F.Cu) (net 3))
 (segment (start 126.6698 101.9302) (end 125.603 101.9302) (width 0.4) (layer F.Cu) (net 3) (status 10))
 (segment (start 126.6698 101.9302) (end 125.603 101.9302) (width 0.4) (layer F.Cu) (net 3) (status 10))
 (segment (start 125.603 101.9302) (end 124.7394 101.0666) (width 0.4) (layer F.Cu) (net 3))
 (segment (start 124.7394 101.0666) (end 124.7394 100.6094) (width 0.4) (layer F.Cu) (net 3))
 (segment (start 124.7394 100.6094) (end 123.7234 99.5934) (width 0.4) (layer F.Cu) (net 3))
 (segment (start 123.7234 99.5934) (end 122.2502 99.5934) (width 0.4) (layer F.Cu) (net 3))
 (segment (start 122.2502 99.5934) (end 121.9708 99.8728) (width 0.4) (layer F.Cu) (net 3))
 (segment (start 121.9708 99.8728) (end 121.9708 101.0742) (width 0.4) (layer F.Cu) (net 3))
 (segment (start 120.7008 96.8248) (end 120.7008 95.6742) (width 0.4) (layer F.Cu) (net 1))
 (segment (start 121.9962 98.1202) (end 120.7008 96.8248) (width 0.4) (layer F.Cu) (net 1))
 (segment (start 124.4854 98.1202) (end 121.9962 98.1202) (width 0.4) (layer F.Cu) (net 1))
 (segment (start 125.7554 99.3902) (end 124.4854 98.1202) (width 0.4) (layer F.Cu) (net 1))
 (segment (start 126.6698 99.3902) (end 125.7554 99.3902) (width 0.4) (layer F.Cu) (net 1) (status 10))
 (segment (start 126.6698 99.3902) (end 125.7554 99.3902) (width 0.4) (layer F.Cu) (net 1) (status 10))
 (segment (start 125.7554 99.3902) (end 124.4854 98.1202) (width 0.4) (layer F.Cu) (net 1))
 (segment (start 124.4854 98.1202) (end 121.9962 98.1202) (width 0.4) (layer F.Cu) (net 1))
 (segment (start 121.9962 98.1202) (end 120.7008 96.8248) (width 0.4) (layer F.Cu) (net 1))
 (segment (start 120.7008 96.8248) (end 120.7008 95.6742) (width 0.4) (layer F.Cu) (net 1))
 (segment (start 130.5306 114.9858) (end 133.477 114.9858) (width 0.5) (layer F.Cu) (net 12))
 (segment (start 130.5306 114.9858) (end 133.477 114.9858) (width 0.5) (layer F.Cu) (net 12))
 (segment (start 130.5306 112.4458) (end 133.477 112.4458) (width 0.5) (layer F.Cu) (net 13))
 (segment (start 130.5306 112.4458) (end 133.477 112.4458) (width 0.5) (layer F.Cu) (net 13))
 (segment (start 116.8146 103.2002) (end 113.3602 99.7458) (width 0.5) (layer F.Cu) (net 14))
 (segment (start 113.3602 99.7458) (end 113.157 99.7458) (width 0.5) (layer F.Cu) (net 14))
 (segment (start 116.8146 103.8098) (end 116.8146 103.2002) (width 0.5) (layer F.Cu) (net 14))
 (segment (start 116.8146 103.8098) (end 116.8146 103.2002) (width 0.5) (layer F.Cu) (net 14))
 (segment (start 113.3602 99.7458) (end 113.157 99.7458) (width 0.5) (layer F.Cu) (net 14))
 (segment (start 116.8146 103.2002) (end 113.3602 99.7458) (width 0.5) (layer F.Cu) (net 14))
 (segment (start 115.9002 106.3498) (end 115.0366 105.4862) (width 0.5) (layer F.Cu) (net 15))
 (segment (start 115.0366 105.4862) (end 115.0366 103.0478) (width 0.5) (layer F.Cu) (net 15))
 (segment (start 115.0366 103.0478) (end 114.2746 102.2858) (width 0.5) (layer F.Cu) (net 15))
 (segment (start 114.2746 102.2858) (end 113.157 102.2858) (width 0.5) (layer F.Cu) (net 15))
 (segment (start 116.8146 106.3498) (end 115.9002 106.3498) (width 0.5) (layer F.Cu) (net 15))
 (segment (start 116.8146 106.3498) (end 115.9002 106.3498) (width 0.5) (layer F.Cu) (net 15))
 (segment (start 114.2746 102.2858) (end 113.157 102.2858) (width 0.5) (layer F.Cu) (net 15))
 (segment (start 115.0366 103.0478) (end 114.2746 102.2858) (width 0.5) (layer F.Cu) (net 15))
 (segment (start 115.0366 105.4862) (end 115.0366 103.0478) (width 0.5) (layer F.Cu) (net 15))
 (segment (start 115.9002 106.3498) (end 115.0366 105.4862) (width 0.5) (layer F.Cu) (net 15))
 (segment (start 118.3386 103.4034) (end 118.3386 104.4702) (width 0.4) (layer F.Cu) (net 2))
 (segment (start 118.3386 104.4702) (end 117.729 105.0798) (width 0.4) (layer F.Cu) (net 2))
 (segment (start 117.729 105.0798) (end 116.8146 105.0798) (width 0.4) (layer F.Cu) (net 2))
 (segment (start 117.729 105.0798) (end 116.8146 105.0798) (width 0.4) (layer F.Cu) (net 2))
 (segment (start 118.3386 104.4702) (end 117.729 105.0798) (width 0.4) (layer F.Cu) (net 2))
 (segment (start 118.3386 103.4034) (end 118.3386 104.4702) (width 0.4) (layer F.Cu) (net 2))
 (segment (start 125.968198 100.6602) (end 124.190198 98.8822) (width 0.4) (layer F.Cu) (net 2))
 (segment (start 124.190198 98.8822) (end 120.3198 98.8822) (width 0.4) (layer F.Cu) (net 2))
 (segment (start 120.3198 98.8822) (end 119.4562 98.0186) (width 0.4) (layer F.Cu) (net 2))
 (segment (start 119.4562 98.0186) (end 115.697 98.0186) (width 0.4) (layer F.Cu) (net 2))
 (segment (start 115.697 98.0186) (end 115.1382 98.5774) (width 0.4) (layer F.Cu) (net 2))
 (segment (start 115.1382 98.5774) (end 115.1382 100.203) (width 0.4) (layer F.Cu) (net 2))
 (segment (start 115.1382 100.203) (end 118.3386 103.4034) (width 0.4) (layer F.Cu) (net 2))
 (segment (start 126.6698 100.6602) (end 125.968198 100.6602) (width 0.4) (layer F.Cu) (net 2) (status 10))
 (segment (start 126.6698 100.6602) (end 128.905 100.6602) (width 0.5) (layer F.Cu) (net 2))
 (segment (start 128.905 100.6602) (end 128.9558 100.6602) (width 0.5) (layer F.Cu) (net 2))
 (segment (start 128.9558 100.6602) (end 130.0226 99.5934) (width 0.5) (layer F.Cu) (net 2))
 (segment (start 130.0226 99.5934) (end 130.0226 97.089) (width 0.5) (layer F.Cu) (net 2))
 (segment (start 130.0226 99.5934) (end 130.0226 97.089) (width 0.5) (layer F.Cu) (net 2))
 (segment (start 128.9558 100.6602) (end 130.0226 99.5934) (width 0.5) (layer F.Cu) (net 2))
 (segment (start 128.905 100.6602) (end 128.9558 100.6602) (width 0.5) (layer F.Cu) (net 2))
 (segment (start 126.6698 100.6602) (end 128.905 100.6602) (width 0.5) (layer F.Cu) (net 2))
 (segment (start 126.6698 100.6602) (end 125.968198 100.6602) (width 0.4) (layer F.Cu) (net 2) (status 10))
 (segment (start 115.1382 100.203) (end 118.3386 103.4034) (width 0.4) (layer F.Cu) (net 2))
 (segment (start 115.1382 98.5774) (end 115.1382 100.203) (width 0.4) (layer F.Cu) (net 2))
 (segment (start 115.697 98.0186) (end 115.1382 98.5774) (width 0.4) (layer F.Cu) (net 2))
 (segment (start 119.4562 98.0186) (end 115.697 98.0186) (width 0.4) (layer F.Cu) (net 2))
 (segment (start 120.3198 98.8822) (end 119.4562 98.0186) (width 0.4) (layer F.Cu) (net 2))
 (segment (start 124.190198 98.8822) (end 120.3198 98.8822) (width 0.4) (layer F.Cu) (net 2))
 (segment (start 125.968198 100.6602) (end 124.190198 98.8822) (width 0.4) (layer F.Cu) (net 2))
 (segment (start 129.5318 105.819) (end 129.8194 105.819) (width 0.5) (layer F.Cu) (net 6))
 (segment (start 129.8194 104.0486) (end 129.8194 105.819) (width 0.5) (layer F.Cu) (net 6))
 (segment (start 129.8194 104.0486) (end 129.8194 105.819) (width 0.5) (layer F.Cu) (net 6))
 (segment (start 129.5318 105.819) (end 129.8194 105.819) (width 0.5) (layer F.Cu) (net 6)))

